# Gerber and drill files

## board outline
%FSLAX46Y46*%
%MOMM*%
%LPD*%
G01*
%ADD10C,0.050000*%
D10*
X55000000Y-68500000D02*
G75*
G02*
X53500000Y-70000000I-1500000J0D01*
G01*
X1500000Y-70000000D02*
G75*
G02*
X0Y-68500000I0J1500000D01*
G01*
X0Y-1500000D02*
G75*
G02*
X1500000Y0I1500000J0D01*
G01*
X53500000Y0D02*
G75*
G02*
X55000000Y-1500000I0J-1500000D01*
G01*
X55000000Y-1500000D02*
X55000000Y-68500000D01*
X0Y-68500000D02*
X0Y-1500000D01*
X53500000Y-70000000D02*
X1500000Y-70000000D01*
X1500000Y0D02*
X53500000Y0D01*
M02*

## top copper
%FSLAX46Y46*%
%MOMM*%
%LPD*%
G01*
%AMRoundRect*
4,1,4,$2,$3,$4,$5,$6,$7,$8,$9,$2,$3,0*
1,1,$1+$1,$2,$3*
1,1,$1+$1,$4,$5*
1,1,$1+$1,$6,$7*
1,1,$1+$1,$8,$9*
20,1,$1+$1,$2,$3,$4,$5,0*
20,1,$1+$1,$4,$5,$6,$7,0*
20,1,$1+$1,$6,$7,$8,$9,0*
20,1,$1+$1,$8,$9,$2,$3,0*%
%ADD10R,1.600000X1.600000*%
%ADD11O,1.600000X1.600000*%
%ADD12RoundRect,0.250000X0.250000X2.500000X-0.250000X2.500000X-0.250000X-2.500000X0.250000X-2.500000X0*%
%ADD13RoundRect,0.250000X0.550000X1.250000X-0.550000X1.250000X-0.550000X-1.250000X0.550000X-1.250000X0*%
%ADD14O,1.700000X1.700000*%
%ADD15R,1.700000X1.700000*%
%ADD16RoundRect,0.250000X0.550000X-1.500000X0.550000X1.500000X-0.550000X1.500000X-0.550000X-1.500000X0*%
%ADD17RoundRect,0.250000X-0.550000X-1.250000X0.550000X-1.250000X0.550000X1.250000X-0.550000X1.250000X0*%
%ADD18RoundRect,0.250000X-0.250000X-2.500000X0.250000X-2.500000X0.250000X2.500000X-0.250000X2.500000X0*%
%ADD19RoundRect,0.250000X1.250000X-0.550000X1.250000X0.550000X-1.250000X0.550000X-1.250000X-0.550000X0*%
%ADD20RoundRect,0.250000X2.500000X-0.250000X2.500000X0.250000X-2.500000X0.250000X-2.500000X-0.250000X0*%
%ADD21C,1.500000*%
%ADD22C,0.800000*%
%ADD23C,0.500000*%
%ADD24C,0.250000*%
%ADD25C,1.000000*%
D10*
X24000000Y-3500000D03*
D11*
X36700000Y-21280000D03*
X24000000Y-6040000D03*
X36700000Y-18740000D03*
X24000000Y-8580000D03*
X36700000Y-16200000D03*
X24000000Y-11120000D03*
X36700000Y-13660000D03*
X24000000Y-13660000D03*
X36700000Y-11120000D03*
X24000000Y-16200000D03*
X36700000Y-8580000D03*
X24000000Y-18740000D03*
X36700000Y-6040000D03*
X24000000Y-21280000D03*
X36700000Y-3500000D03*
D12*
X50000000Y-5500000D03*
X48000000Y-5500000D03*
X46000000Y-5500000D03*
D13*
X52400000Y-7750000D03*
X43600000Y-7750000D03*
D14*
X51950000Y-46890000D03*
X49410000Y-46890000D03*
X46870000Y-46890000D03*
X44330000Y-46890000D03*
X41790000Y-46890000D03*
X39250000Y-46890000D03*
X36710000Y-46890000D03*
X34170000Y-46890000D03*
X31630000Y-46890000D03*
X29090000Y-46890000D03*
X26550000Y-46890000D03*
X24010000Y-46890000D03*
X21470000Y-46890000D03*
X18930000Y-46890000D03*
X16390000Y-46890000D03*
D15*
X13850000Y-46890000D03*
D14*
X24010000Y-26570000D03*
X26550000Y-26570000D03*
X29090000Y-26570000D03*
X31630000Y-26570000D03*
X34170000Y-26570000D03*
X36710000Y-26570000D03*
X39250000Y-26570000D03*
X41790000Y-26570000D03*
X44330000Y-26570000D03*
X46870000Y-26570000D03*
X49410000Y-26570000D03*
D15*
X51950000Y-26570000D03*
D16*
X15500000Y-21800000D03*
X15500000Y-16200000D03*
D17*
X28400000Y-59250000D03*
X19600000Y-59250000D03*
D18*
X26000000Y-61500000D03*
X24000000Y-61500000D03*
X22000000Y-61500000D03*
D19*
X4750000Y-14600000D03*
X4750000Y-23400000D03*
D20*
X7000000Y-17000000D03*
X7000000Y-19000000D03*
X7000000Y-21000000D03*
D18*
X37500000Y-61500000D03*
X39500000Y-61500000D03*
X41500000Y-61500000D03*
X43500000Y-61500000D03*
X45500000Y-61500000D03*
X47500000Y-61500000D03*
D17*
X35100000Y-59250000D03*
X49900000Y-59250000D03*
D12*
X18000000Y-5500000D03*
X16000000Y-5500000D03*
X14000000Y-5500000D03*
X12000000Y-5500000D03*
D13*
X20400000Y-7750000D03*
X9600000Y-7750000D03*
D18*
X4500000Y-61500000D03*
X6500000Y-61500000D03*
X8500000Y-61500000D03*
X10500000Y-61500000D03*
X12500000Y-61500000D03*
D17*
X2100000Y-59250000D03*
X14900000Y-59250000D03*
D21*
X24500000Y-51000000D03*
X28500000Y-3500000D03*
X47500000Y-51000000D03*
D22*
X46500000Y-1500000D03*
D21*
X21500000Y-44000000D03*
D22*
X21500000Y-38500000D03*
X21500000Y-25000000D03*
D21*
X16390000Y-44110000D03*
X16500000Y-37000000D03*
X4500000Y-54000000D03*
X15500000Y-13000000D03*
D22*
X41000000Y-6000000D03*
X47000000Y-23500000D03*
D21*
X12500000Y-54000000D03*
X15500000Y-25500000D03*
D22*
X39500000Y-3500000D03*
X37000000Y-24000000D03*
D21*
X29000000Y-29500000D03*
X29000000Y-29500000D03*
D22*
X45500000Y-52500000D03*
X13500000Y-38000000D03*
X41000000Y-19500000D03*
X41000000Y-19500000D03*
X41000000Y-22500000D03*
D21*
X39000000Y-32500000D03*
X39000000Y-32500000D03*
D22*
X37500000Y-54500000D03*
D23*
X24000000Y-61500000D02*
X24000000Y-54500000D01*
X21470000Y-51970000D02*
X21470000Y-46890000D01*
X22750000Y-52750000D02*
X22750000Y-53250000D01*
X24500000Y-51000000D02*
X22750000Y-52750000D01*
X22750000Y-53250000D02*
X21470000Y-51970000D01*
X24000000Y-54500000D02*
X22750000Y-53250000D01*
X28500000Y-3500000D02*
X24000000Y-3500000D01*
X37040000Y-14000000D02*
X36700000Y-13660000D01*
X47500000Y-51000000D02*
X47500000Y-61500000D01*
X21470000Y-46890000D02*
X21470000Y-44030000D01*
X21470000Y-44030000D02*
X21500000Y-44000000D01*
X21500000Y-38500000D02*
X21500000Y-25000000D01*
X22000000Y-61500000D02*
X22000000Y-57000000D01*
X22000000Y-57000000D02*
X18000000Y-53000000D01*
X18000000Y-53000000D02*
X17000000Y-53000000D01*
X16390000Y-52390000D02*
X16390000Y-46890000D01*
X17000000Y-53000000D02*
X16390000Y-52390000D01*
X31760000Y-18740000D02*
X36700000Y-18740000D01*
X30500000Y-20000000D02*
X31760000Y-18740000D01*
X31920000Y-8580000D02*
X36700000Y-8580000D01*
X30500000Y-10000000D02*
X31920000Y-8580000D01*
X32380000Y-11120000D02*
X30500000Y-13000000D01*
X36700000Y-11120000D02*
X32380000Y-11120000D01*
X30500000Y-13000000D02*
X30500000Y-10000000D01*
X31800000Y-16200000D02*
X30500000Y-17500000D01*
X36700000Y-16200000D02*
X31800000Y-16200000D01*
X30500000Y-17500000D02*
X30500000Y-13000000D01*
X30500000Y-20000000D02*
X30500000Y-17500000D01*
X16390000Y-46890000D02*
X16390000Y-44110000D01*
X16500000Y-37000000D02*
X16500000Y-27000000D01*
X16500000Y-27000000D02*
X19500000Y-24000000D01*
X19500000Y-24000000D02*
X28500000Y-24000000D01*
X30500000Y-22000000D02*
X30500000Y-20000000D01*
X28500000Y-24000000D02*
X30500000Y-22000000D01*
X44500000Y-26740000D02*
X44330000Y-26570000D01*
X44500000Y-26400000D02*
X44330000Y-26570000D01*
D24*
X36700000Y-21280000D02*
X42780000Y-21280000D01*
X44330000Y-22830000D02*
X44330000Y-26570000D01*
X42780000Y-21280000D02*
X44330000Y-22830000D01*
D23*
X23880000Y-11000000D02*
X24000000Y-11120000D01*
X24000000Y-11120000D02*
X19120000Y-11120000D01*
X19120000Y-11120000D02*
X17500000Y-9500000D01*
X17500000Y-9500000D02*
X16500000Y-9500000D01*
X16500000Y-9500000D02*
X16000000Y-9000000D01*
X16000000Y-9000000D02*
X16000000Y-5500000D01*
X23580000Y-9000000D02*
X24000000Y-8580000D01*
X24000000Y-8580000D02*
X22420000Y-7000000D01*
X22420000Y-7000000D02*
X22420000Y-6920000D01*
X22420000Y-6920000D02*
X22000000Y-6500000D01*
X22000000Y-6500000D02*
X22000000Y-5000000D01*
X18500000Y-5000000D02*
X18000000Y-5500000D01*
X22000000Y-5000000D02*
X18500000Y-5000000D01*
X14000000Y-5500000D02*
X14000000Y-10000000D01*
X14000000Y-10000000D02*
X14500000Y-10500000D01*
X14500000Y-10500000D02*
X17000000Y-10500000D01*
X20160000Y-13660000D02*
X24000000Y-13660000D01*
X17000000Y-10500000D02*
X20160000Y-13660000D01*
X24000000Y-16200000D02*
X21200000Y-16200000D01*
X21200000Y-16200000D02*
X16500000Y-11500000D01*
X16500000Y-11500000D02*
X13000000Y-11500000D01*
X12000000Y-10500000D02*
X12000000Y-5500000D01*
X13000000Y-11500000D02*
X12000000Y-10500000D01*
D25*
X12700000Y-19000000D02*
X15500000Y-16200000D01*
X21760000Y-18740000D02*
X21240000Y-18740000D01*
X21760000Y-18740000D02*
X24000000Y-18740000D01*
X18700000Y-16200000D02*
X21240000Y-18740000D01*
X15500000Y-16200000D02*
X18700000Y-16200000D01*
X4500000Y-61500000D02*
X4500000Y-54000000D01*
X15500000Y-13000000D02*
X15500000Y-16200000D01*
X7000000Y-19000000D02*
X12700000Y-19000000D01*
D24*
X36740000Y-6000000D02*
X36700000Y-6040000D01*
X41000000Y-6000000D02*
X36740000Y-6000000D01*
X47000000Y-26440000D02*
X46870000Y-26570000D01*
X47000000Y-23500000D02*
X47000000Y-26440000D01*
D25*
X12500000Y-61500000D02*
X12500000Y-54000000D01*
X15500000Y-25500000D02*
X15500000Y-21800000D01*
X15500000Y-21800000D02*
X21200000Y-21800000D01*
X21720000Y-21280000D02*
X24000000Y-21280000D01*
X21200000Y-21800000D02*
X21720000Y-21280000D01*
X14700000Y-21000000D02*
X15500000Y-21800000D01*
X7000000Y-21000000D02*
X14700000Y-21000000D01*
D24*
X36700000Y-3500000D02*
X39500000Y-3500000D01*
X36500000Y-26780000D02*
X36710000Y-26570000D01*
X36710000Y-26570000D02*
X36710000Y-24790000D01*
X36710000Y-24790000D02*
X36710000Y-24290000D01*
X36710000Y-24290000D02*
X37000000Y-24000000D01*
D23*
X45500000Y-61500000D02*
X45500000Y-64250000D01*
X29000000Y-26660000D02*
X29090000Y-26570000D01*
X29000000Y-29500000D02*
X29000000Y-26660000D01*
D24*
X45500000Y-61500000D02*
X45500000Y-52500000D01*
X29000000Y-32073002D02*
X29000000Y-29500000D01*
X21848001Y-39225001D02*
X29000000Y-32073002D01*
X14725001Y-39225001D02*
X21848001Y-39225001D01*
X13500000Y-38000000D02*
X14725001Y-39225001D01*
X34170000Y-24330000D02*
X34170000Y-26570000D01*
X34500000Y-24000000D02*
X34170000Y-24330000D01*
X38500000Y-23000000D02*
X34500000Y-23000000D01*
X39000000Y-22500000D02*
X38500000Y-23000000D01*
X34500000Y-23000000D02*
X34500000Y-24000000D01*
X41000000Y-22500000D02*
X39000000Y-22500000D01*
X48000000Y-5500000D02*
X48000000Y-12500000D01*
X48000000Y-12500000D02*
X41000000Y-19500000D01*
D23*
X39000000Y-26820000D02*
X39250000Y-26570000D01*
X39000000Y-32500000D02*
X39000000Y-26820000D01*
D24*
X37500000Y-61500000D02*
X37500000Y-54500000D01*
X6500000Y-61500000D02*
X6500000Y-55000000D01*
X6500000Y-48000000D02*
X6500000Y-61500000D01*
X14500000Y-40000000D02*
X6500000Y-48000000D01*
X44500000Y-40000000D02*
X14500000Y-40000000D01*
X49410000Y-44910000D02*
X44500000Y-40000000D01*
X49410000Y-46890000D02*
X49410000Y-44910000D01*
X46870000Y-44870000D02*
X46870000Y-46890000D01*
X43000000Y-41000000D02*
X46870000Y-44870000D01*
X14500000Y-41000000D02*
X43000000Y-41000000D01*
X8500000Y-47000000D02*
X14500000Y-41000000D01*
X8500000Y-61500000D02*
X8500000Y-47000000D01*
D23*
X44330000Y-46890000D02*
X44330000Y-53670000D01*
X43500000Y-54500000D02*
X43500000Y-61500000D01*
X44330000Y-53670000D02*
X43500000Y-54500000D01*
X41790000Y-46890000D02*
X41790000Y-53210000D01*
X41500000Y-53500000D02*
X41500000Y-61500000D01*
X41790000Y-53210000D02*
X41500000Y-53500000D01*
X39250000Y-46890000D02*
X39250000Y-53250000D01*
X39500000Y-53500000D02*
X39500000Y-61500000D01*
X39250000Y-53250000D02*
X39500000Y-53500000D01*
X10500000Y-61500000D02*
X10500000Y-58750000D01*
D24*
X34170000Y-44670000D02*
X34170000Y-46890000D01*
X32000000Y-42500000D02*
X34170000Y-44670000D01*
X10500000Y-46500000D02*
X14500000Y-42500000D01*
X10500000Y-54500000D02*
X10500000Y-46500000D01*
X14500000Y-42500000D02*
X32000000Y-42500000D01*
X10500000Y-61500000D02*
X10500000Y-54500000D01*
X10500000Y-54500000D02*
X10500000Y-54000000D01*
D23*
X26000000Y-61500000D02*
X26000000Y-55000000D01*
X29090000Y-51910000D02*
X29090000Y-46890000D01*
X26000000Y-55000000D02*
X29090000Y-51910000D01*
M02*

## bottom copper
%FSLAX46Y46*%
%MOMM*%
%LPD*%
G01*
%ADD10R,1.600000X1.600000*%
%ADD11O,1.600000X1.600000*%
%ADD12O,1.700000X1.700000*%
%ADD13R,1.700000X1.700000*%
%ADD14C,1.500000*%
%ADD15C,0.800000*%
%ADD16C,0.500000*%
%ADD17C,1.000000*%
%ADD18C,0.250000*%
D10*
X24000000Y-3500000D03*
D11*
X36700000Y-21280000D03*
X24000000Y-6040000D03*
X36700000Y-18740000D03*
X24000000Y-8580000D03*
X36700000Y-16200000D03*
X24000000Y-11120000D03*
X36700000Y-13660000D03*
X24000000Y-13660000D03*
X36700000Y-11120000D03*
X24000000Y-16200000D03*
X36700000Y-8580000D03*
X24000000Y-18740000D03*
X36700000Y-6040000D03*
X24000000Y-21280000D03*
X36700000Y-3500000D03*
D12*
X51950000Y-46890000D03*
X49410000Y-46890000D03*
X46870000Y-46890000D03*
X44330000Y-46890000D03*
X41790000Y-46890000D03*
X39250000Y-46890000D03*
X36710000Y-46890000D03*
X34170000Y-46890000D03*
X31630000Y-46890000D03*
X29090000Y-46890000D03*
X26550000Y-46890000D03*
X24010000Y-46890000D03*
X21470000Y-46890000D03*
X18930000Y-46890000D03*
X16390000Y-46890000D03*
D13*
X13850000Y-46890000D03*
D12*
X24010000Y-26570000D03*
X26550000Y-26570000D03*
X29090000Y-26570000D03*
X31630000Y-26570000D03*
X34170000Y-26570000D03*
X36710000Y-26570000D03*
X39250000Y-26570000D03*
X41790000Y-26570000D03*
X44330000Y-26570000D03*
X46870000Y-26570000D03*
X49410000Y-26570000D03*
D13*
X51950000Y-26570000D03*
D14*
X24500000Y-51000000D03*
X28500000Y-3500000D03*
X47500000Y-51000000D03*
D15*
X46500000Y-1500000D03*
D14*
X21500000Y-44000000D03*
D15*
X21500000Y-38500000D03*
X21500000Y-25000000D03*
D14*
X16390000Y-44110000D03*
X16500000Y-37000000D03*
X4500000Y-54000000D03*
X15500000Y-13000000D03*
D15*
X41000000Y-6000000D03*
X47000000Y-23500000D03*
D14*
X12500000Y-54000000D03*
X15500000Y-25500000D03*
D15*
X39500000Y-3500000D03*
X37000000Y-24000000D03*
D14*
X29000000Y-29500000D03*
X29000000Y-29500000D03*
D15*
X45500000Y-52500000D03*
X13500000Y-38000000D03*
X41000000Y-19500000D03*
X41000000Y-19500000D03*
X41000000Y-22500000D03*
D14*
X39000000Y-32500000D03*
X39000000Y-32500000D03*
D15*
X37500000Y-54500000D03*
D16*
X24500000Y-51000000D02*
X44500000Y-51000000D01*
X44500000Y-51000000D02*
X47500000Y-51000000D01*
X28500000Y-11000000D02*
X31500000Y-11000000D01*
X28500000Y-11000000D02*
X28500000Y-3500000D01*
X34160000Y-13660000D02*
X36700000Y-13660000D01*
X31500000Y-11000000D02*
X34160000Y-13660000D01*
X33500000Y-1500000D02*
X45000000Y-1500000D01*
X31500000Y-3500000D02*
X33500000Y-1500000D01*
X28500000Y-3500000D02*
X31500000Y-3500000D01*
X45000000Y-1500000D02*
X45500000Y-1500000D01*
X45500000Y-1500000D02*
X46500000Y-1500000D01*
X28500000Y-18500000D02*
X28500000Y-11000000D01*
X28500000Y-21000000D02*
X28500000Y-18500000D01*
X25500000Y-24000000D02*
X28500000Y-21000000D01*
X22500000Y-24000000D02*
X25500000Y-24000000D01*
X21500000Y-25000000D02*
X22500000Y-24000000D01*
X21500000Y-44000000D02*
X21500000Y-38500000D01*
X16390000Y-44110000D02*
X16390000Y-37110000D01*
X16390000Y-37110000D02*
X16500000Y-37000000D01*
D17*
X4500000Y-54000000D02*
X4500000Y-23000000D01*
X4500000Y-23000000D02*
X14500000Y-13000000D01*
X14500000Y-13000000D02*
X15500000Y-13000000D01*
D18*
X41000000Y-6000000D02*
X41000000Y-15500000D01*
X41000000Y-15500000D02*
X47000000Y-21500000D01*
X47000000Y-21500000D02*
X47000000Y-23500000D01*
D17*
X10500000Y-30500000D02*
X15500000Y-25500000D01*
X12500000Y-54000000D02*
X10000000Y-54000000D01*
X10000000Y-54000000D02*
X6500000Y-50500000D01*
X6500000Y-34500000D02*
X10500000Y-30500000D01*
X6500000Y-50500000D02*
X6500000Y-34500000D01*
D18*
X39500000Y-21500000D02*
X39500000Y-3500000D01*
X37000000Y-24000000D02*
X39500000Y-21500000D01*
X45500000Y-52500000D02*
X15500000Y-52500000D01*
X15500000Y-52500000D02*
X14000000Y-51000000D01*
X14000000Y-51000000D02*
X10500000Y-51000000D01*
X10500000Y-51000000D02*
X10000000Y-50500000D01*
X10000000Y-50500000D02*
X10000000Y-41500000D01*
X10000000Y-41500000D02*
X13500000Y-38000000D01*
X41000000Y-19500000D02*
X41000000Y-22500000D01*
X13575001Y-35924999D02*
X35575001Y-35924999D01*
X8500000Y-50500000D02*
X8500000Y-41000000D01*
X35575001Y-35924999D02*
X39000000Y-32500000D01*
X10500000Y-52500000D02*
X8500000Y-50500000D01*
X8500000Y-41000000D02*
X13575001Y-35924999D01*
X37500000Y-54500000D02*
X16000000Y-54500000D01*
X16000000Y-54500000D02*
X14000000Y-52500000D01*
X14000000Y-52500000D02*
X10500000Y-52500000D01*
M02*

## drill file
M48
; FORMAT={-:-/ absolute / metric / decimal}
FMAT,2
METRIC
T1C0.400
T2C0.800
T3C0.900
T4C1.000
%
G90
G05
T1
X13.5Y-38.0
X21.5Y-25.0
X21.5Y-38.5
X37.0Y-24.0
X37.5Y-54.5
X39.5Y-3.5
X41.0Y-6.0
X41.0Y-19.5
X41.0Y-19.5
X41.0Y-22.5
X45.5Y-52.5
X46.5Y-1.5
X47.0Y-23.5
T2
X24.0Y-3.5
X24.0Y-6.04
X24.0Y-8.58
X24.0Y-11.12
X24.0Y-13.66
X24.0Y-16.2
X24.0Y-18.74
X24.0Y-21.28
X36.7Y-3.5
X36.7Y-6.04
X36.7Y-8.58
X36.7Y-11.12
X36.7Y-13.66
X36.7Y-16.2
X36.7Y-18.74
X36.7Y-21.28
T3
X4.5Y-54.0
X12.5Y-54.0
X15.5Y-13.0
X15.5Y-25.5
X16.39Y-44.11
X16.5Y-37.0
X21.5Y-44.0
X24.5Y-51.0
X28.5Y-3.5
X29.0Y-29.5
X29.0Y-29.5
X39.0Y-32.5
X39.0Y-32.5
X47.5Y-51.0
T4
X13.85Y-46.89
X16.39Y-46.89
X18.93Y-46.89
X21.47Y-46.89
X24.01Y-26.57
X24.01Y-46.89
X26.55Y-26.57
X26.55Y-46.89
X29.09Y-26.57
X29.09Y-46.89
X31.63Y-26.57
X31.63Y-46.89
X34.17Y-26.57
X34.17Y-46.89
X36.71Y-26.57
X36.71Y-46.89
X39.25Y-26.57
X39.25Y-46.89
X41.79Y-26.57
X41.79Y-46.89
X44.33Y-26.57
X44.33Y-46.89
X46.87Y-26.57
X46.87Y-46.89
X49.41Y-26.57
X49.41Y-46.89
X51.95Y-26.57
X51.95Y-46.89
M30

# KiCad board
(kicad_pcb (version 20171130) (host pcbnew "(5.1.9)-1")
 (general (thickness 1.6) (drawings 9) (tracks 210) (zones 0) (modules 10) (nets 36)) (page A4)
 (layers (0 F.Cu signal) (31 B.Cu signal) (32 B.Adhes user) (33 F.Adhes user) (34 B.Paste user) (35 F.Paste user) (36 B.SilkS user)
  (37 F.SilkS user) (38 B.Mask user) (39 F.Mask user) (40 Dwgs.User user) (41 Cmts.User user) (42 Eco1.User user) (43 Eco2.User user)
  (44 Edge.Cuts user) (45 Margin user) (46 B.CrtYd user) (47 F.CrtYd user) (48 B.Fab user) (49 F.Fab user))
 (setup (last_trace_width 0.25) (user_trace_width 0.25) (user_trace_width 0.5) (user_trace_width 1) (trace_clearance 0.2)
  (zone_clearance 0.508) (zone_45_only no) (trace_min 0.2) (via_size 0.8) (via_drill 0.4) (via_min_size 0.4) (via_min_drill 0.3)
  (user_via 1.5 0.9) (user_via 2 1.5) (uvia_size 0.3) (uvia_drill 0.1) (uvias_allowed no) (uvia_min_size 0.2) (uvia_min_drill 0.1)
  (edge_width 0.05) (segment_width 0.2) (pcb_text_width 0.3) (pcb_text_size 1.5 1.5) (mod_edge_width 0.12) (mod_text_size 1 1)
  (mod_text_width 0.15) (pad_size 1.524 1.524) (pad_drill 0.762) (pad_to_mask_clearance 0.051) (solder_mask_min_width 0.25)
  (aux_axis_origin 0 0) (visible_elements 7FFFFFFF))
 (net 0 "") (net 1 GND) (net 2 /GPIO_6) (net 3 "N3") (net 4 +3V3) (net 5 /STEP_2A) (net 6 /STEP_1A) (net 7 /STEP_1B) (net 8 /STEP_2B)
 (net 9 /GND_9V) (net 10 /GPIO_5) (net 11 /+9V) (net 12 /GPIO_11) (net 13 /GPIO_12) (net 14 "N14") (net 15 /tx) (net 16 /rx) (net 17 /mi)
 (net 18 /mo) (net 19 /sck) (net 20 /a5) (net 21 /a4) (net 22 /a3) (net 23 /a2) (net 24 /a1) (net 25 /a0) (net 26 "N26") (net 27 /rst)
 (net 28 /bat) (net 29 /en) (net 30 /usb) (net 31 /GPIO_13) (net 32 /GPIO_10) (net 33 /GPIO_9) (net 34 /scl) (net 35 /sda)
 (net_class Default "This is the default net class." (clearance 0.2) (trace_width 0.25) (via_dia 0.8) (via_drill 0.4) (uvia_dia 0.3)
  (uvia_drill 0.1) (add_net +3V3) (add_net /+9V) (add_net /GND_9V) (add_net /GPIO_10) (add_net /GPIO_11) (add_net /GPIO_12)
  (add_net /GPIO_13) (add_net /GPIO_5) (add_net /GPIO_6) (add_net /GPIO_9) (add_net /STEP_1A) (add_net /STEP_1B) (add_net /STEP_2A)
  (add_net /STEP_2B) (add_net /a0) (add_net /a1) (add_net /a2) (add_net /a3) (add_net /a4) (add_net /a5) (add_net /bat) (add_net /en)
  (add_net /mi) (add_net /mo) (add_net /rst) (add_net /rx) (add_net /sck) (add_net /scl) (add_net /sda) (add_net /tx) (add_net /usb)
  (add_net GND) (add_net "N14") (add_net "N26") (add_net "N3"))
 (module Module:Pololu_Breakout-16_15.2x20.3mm (layer F.Cu) (at 24 3.5)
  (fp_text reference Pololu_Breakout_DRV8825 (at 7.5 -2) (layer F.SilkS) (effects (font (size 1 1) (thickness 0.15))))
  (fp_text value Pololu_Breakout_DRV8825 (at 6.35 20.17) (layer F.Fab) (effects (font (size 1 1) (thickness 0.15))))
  (pad 1 thru_hole rect (at 0 0) (size 1.6 1.6) (drill 0.8) (layers *.Cu *.Mask) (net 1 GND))
  (pad 9 thru_hole oval (at 12.7 17.78) (size 1.6 1.6) (drill 0.8) (layers *.Cu *.Mask) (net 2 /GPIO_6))
  (pad 2 thru_hole oval (at 0 2.54) (size 1.6 1.6) (drill 0.8) (layers *.Cu *.Mask) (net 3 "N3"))
  (pad 10 thru_hole oval (at 12.7 15.24) (size 1.6 1.6) (drill 0.8) (layers *.Cu *.Mask) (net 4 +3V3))
  (pad 3 thru_hole oval (at 0 5.08) (size 1.6 1.6) (drill 0.8) (layers *.Cu *.Mask) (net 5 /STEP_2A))
  (pad 11 thru_hole oval (at 12.7 12.7) (size 1.6 1.6) (drill 0.8) (layers *.Cu *.Mask) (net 4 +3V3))
  (pad 4 thru_hole oval (at 0 7.62) (size 1.6 1.6) (drill 0.8) (layers *.Cu *.Mask) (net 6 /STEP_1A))
  (pad 12 thru_hole oval (at 12.7 10.16) (size 1.6 1.6) (drill 0.8) (layers *.Cu *.Mask) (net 1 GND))
  (pad 5 thru_hole oval (at 0 10.16) (size 1.6 1.6) (drill 0.8) (layers *.Cu *.Mask) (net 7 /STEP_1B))
  (pad 13 thru_hole oval (at 12.7 7.62) (size 1.6 1.6) (drill 0.8) (layers *.Cu *.Mask) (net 4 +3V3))
  (pad 6 thru_hole oval (at 0 12.7) (size 1.6 1.6) (drill 0.8) (layers *.Cu *.Mask) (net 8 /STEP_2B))
  (pad 14 thru_hole oval (at 12.7 5.08) (size 1.6 1.6) (drill 0.8) (layers *.Cu *.Mask) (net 4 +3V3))
  (pad 7 thru_hole oval (at 0 15.24) (size 1.6 1.6) (drill 0.8) (layers *.Cu *.Mask) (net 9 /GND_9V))
  (pad 15 thru_hole oval (at 12.7 2.54) (size 1.6 1.6) (drill 0.8) (layers *.Cu *.Mask) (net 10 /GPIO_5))
  (pad 8 thru_hole oval (at 0 17.78) (size 1.6 1.6) (drill 0.8) (layers *.Cu *.Mask) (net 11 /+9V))
  (pad 16 thru_hole oval (at 12.7 0) (size 1.6 1.6) (drill 0.8) (layers *.Cu *.Mask) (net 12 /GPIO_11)))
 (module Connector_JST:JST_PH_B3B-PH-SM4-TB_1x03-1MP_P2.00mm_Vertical (layer F.Cu) (at 48 6 180)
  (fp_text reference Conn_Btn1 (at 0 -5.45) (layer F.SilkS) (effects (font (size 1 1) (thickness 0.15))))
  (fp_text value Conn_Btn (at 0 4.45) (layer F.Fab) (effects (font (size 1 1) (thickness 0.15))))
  (pad 1 smd roundrect (at -2 0.5 180) (size 1 5.5) (layers F.Cu F.Paste F.Mask) (roundrect_rratio 0.25) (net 1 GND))
  (pad 2 smd roundrect (at 0 0.5 180) (size 1 5.5) (layers F.Cu F.Paste F.Mask) (roundrect_rratio 0.25) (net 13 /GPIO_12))
  (pad 3 smd roundrect (at 2 0.5 180) (size 1 5.5) (layers F.Cu F.Paste F.Mask) (roundrect_rratio 0.25))
  (pad MP smd roundrect (at -4.4 -1.75 180) (size 1.6 3) (layers F.Cu F.Paste F.Mask) (roundrect_rratio 0.15625))
  (pad MP smd roundrect (at 4.4 -1.75 180) (size 1.6 3) (layers F.Cu F.Paste F.Mask) (roundrect_rratio 0.15625)))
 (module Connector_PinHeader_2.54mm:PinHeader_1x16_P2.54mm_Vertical (layer F.Cu) (at 13.85 46.89 90)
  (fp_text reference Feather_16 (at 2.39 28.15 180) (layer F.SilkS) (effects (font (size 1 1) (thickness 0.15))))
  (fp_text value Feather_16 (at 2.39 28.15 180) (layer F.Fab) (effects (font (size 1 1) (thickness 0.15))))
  (pad 16 thru_hole oval (at 0 38.1 90) (size 1.7 1.7) (drill 1) (layers *.Cu *.Mask) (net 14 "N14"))
  (pad 15 thru_hole oval (at 0 35.56 90) (size 1.7 1.7) (drill 1) (layers *.Cu *.Mask) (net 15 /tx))
  (pad 14 thru_hole oval (at 0 33.02 90) (size 1.7 1.7) (drill 1) (layers *.Cu *.Mask) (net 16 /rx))
  (pad 13 thru_hole oval (at 0 30.48 90) (size 1.7 1.7) (drill 1) (layers *.Cu *.Mask) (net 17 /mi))
  (pad 12 thru_hole oval (at 0 27.94 90) (size 1.7 1.7) (drill 1) (layers *.Cu *.Mask) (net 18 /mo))
  (pad 11 thru_hole oval (at 0 25.4 90) (size 1.7 1.7) (drill 1) (layers *.Cu *.Mask) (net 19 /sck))
  (pad 10 thru_hole oval (at 0 22.86 90) (size 1.7 1.7) (drill 1) (layers *.Cu *.Mask) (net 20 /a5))
  (pad 9 thru_hole oval (at 0 20.32 90) (size 1.7 1.7) (drill 1) (layers *.Cu *.Mask) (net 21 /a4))
  (pad 8 thru_hole oval (at 0 17.78 90) (size 1.7 1.7) (drill 1) (layers *.Cu *.Mask) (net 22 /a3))
  (pad 7 thru_hole oval (at 0 15.24 90) (size 1.7 1.7) (drill 1) (layers *.Cu *.Mask) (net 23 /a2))
  (pad 6 thru_hole oval (at 0 12.7 90) (size 1.7 1.7) (drill 1) (layers *.Cu *.Mask) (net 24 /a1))
  (pad 5 thru_hole oval (at 0 10.16 90) (size 1.7 1.7) (drill 1) (layers *.Cu *.Mask) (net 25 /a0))
  (pad 4 thru_hole oval (at 0 7.62 90) (size 1.7 1.7) (drill 1) (layers *.Cu *.Mask) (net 1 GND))
  (pad 3 thru_hole oval (at 0 5.08 90) (size 1.7 1.7) (drill 1) (layers *.Cu *.Mask) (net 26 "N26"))
  (pad 2 thru_hole oval (at 0 2.54 90) (size 1.7 1.7) (drill 1) (layers *.Cu *.Mask) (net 4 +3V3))
  (pad 1 thru_hole rect (at 0 0 90) (size 1.7 1.7) (drill 1) (layers *.Cu *.Mask) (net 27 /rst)))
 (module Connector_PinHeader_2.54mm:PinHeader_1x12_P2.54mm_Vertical (layer F.Cu) (at 51.95 26.57 270)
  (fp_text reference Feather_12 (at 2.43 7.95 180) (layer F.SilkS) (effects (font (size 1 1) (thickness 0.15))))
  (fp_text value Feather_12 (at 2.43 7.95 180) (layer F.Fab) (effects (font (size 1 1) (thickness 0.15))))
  (pad 12 thru_hole oval (at 0 27.94 270) (size 1.7 1.7) (drill 1) (layers *.Cu *.Mask) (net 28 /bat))
  (pad 11 thru_hole oval (at 0 25.4 270) (size 1.7 1.7) (drill 1) (layers *.Cu *.Mask) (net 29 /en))
  (pad 10 thru_hole oval (at 0 22.86 270) (size 1.7 1.7) (drill 1) (layers *.Cu *.Mask) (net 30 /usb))
  (pad 9 thru_hole oval (at 0 20.32 270) (size 1.7 1.7) (drill 1) (layers *.Cu *.Mask) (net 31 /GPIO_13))
  (pad 8 thru_hole oval (at 0 17.78 270) (size 1.7 1.7) (drill 1) (layers *.Cu *.Mask) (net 13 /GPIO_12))
  (pad 7 thru_hole oval (at 0 15.24 270) (size 1.7 1.7) (drill 1) (layers *.Cu *.Mask) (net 12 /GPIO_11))
  (pad 6 thru_hole oval (at 0 12.7 270) (size 1.7 1.7) (drill 1) (layers *.Cu *.Mask) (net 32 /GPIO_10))
  (pad 5 thru_hole oval (at 0 10.16 270) (size 1.7 1.7) (drill 1) (layers *.Cu *.Mask) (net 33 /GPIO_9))
  (pad 4 thru_hole oval (at 0 7.62 270) (size 1.7 1.7) (drill 1) (layers *.Cu *.Mask) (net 2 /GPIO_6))
  (pad 3 thru_hole oval (at 0 5.08 270) (size 1.7 1.7) (drill 1) (layers *.Cu *.Mask) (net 10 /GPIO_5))
  (pad 2 thru_hole oval (at 0 2.54 270) (size 1.7 1.7) (drill 1) (layers *.Cu *.Mask) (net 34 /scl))
  (pad 1 thru_hole rect (at 0 0 270) (size 1.7 1.7) (drill 1) (layers *.Cu *.Mask) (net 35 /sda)))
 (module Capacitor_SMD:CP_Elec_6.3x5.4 (layer F.Cu) (at 15.5 19 90)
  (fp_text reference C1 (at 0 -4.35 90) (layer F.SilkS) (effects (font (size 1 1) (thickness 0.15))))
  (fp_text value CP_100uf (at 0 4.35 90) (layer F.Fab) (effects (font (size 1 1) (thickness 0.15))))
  (pad 1 smd roundrect (at -2.8 0 90) (size 3.5 1.6) (layers F.Cu F.Paste F.Mask) (roundrect_rratio 0.15625) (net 11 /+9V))
  (pad 2 smd roundrect (at 2.8 0 90) (size 3.5 1.6) (layers F.Cu F.Paste F.Mask) (roundrect_rratio 0.15625) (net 9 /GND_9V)))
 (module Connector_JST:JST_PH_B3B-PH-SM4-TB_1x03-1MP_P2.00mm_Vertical (layer F.Cu) (at 24 61)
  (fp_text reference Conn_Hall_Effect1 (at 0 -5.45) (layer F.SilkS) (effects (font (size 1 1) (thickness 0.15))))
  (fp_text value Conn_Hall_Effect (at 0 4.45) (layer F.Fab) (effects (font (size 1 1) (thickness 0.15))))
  (pad MP smd roundrect (at 4.4 -1.75) (size 1.6 3) (layers F.Cu F.Paste F.Mask) (roundrect_rratio 0.15625))
  (pad MP smd roundrect (at -4.4 -1.75) (size 1.6 3) (layers F.Cu F.Paste F.Mask) (roundrect_rratio 0.15625))
  (pad 3 smd roundrect (at 2 0.5) (size 1 5.5) (layers F.Cu F.Paste F.Mask) (roundrect_rratio 0.25) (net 23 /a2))
  (pad 2 smd roundrect (at 0 0.5) (size 1 5.5) (layers F.Cu F.Paste F.Mask) (roundrect_rratio 0.25) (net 1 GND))
  (pad 1 smd roundrect (at -2 0.5) (size 1 5.5) (layers F.Cu F.Paste F.Mask) (roundrect_rratio 0.25) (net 4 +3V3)))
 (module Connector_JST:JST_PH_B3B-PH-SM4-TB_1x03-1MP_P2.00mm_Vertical (layer F.Cu) (at 6.5 19 90)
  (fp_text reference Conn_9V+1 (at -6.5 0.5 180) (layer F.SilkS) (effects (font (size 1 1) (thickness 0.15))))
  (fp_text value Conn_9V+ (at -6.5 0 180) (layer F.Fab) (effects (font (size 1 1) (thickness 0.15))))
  (pad MP smd roundrect (at 4.4 -1.75 90) (size 1.6 3) (layers F.Cu F.Paste F.Mask) (roundrect_rratio 0.15625))
  (pad MP smd roundrect (at -4.4 -1.75 90) (size 1.6 3) (layers F.Cu F.Paste F.Mask) (roundrect_rratio 0.15625))
  (pad 3 smd roundrect (at 2 0.5 90) (size 1 5.5) (layers F.Cu F.Paste F.Mask) (roundrect_rratio 0.25))
  (pad 2 smd roundrect (at 0 0.5 90) (size 1 5.5) (layers F.Cu F.Paste F.Mask) (roundrect_rratio 0.25) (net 9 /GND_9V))
  (pad 1 smd roundrect (at -2 0.5 90) (size 1 5.5) (layers F.Cu F.Paste F.Mask) (roundrect_rratio 0.25) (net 11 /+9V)))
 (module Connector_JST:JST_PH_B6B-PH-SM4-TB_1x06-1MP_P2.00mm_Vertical (layer F.Cu) (at 42.5 61)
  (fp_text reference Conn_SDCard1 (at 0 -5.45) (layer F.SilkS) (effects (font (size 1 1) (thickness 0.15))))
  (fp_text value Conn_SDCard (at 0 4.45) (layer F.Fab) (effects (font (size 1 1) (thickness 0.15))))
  (pad 1 smd roundrect (at -5 0.5) (size 1 5.5) (layers F.Cu F.Paste F.Mask) (roundrect_rratio 0.25) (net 32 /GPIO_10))
  (pad 2 smd roundrect (at -3 0.5) (size 1 5.5) (layers F.Cu F.Paste F.Mask) (roundrect_rratio 0.25) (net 19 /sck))
  (pad 3 smd roundrect (at -1 0.5) (size 1 5.5) (layers F.Cu F.Paste F.Mask) (roundrect_rratio 0.25) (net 18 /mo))
  (pad 4 smd roundrect (at 1 0.5) (size 1 5.5) (layers F.Cu F.Paste F.Mask) (roundrect_rratio 0.25) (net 17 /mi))
  (pad 5 smd roundrect (at 3 0.5) (size 1 5.5) (layers F.Cu F.Paste F.Mask) (roundrect_rratio 0.25) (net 30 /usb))
  (pad 6 smd roundrect (at 5 0.5) (size 1 5.5) (layers F.Cu F.Paste F.Mask) (roundrect_rratio 0.25) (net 1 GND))
  (pad MP smd roundrect (at -7.4 -1.75) (size 1.6 3) (layers F.Cu F.Paste F.Mask) (roundrect_rratio 0.15625))
  (pad MP smd roundrect (at 7.4 -1.75) (size 1.6 3) (layers F.Cu F.Paste F.Mask) (roundrect_rratio 0.15625)))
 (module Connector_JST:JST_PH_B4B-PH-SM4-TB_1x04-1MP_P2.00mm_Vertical (layer F.Cu) (at 15 6 180)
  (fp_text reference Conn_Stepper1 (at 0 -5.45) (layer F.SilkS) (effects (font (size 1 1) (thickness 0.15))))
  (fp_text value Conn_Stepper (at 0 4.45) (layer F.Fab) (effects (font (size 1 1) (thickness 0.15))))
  (pad 1 smd roundrect (at -3 0.5 180) (size 1 5.5) (layers F.Cu F.Paste F.Mask) (roundrect_rratio 0.25) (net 5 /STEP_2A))
  (pad 2 smd roundrect (at -1 0.5 180) (size 1 5.5) (layers F.Cu F.Paste F.Mask) (roundrect_rratio 0.25) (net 6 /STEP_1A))
  (pad 3 smd roundrect (at 1 0.5 180) (size 1 5.5) (layers F.Cu F.Paste F.Mask) (roundrect_rratio 0.25) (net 7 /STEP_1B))
  (pad 4 smd roundrect (at 3 0.5 180) (size 1 5.5) (layers F.Cu F.Paste F.Mask) (roundrect_rratio 0.25) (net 8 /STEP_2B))
  (pad MP smd roundrect (at -5.4 -1.75 180) (size 1.6 3) (layers F.Cu F.Paste F.Mask) (roundrect_rratio 0.15625))
  (pad MP smd roundrect (at 5.4 -1.75 180) (size 1.6 3) (layers F.Cu F.Paste F.Mask) (roundrect_rratio 0.15625)))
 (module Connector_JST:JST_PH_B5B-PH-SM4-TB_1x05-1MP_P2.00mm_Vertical (layer F.Cu) (at 8.5 61)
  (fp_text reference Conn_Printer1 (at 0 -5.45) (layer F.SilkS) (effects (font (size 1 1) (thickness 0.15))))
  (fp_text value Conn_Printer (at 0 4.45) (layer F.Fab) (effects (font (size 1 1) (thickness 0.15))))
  (pad 1 smd roundrect (at -4 0.5) (size 1 5.5) (layers F.Cu F.Paste F.Mask) (roundrect_rratio 0.25) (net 9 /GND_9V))
  (pad 2 smd roundrect (at -2 0.5) (size 1 5.5) (layers F.Cu F.Paste F.Mask) (roundrect_rratio 0.25) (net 15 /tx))
  (pad 3 smd roundrect (at 0 0.5) (size 1 5.5) (layers F.Cu F.Paste F.Mask) (roundrect_rratio 0.25) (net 16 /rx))
  (pad 4 smd roundrect (at 2 0.5) (size 1 5.5) (layers F.Cu F.Paste F.Mask) (roundrect_rratio 0.25) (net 21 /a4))
  (pad 5 smd roundrect (at 4 0.5) (size 1 5.5) (layers F.Cu F.Paste F.Mask) (roundrect_rratio 0.25) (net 11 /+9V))
  (pad MP smd roundrect (at -6.4 -1.75) (size 1.6 3) (layers F.Cu F.Paste F.Mask) (roundrect_rratio 0.15625))
  (pad MP smd roundrect (at 6.4 -1.75) (size 1.6 3) (layers F.Cu F.Paste F.Mask) (roundrect_rratio 0.15625)))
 (gr_arc (start 53.5 68.5) (end 53.5 70) (angle -90) (layer Edge.Cuts) (width 0.05))
 (gr_arc (start 1.5 68.5) (end 0 68.5) (angle -90) (layer Edge.Cuts) (width 0.05))
 (gr_arc (start 1.5 1.5) (end 1.5 0) (angle -90) (layer Edge.Cuts) (width 0.05))
 (gr_arc (start 53.5 1.5) (end 55 1.5) (angle -90) (layer Edge.Cuts) (width 0.05))
 (gr_line (start 55 1.5) (end 55 68.5) (layer Edge.Cuts) (width 0.05))
 (gr_line (start 0 68.5) (end 0 1.5) (layer Edge.Cuts) (width 0.05))
 (gr_line (start 53.5 70) (end 1.5 70) (layer Edge.Cuts) (width 0.05))
 (gr_line (start 1.5 0) (end 53.5 0) (layer Edge.Cuts) (width 0.05))
 (segment (start 24 61.5) (end 24 54.5) (width 0.5) (layer F.Cu) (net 1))
 (segment (start 21.47 51.97) (end 21.47 46.89) (width 0.5) (layer F.Cu) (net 1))
 (via (at 24.5 51) (size 1.5) (drill 0.9) (layers F.Cu B.Cu) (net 1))
 (segment (start 22.75 52.75) (end 22.75 53.25) (width 0.5) (layer F.Cu) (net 1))
 (segment (start 24.5 51) (end 22.75 52.75) (width 0.5) (layer F.Cu) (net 1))
 (segment (start 22.75 53.25) (end 21.47 51.97) (width 0.5) (layer F.Cu) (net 1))
 (segment (start 24 54.5) (end 22.75 53.25) (width 0.5) (layer F.Cu) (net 1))
 (segment (start 24.5 51) (end 44.5 51) (width 0.5) (layer B.Cu) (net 1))
 (via (at 28.5 3.5) (size 1.5) (drill 0.9) (layers F.Cu B.Cu) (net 1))
 (segment (start 28.5 3.5) (end 24 3.5) (width 0.5) (layer F.Cu) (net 1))
 (segment (start 37.04 14) (end 36.7 13.66) (width 0.5) (layer F.Cu) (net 1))
 (segment (start 44.5 51) (end 47.5 51) (width 0.5) (layer B.Cu) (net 1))
 (via (at 47.5 51) (size 1.5) (drill 0.9) (layers F.Cu B.Cu) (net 1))
 (segment (start 47.5 51) (end 47.5 61.5) (width 0.5) (layer F.Cu) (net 1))
 (segment (start 28.5 11) (end 31.5 11) (width 0.5) (layer B.Cu) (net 1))
 (segment (start 28.5 11) (end 28.5 3.5) (width 0.5) (layer B.Cu) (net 1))
 (segment (start 34.16 13.66) (end 36.7 13.66) (width 0.5) (layer B.Cu) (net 1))
 (segment (start 31.5 11) (end 34.16 13.66) (width 0.5) (layer B.Cu) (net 1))
 (segment (start 33.5 1.5) (end 45 1.5) (width 0.5) (layer B.Cu) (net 1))
 (segment (start 31.5 3.5) (end 33.5 1.5) (width 0.5) (layer B.Cu) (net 1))
 (segment (start 28.5 3.5) (end 31.5 3.5) (width 0.5) (layer B.Cu) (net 1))
 (segment (start 45 1.5) (end 45.5 1.5) (width 0.5) (layer B.Cu) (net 1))
 (segment (start 45.5 1.5) (end 46.5 1.5) (width 0.5) (layer B.Cu) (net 1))
 (via (at 46.5 1.5) (size 0.8) (drill 0.4) (layers F.Cu B.Cu) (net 1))
 (segment (start 21.47 46.89) (end 21.47 44.03) (width 0.5) (layer F.Cu) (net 1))
 (via (at 21.5 44) (size 1.5) (drill 0.9) (layers F.Cu B.Cu) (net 1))
 (segment (start 21.47 44.03) (end 21.5 44) (width 0.5) (layer F.Cu) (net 1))
 (segment (start 28.5 18.5) (end 28.5 11) (width 0.5) (layer B.Cu) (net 1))
 (segment (start 28.5 21) (end 28.5 18.5) (width 0.5) (layer B.Cu) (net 1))
 (segment (start 25.5 24) (end 28.5 21) (width 0.5) (layer B.Cu) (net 1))
 (segment (start 22.5 24) (end 25.5 24) (width 0.5) (layer B.Cu) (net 1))
 (segment (start 21.5 25) (end 22.5 24) (width 0.5) (layer B.Cu) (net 1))
 (segment (start 21.5 44) (end 21.5 38.5) (width 0.5) (layer B.Cu) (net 1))
 (via (at 21.5 38.5) (size 0.8) (drill 0.4) (layers F.Cu B.Cu) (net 1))
 (segment (start 21.5 38.5) (end 21.5 25) (width 0.5) (layer F.Cu) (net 1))
 (via (at 21.5 25) (size 0.8) (drill 0.4) (layers F.Cu B.Cu) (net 1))
 (segment (start 22 61.5) (end 22 57) (width 0.5) (layer F.Cu) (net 4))
 (segment (start 22 57) (end 18 53) (width 0.5) (layer F.Cu) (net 4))
 (segment (start 18 53) (end 17 53) (width 0.5) (layer F.Cu) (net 4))
 (segment (start 16.39 52.39) (end 16.39 46.89) (width 0.5) (layer F.Cu) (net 4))
 (segment (start 17 53) (end 16.39 52.39) (width 0.5) (layer F.Cu) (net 4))
 (segment (start 31.76 18.74) (end 36.7 18.74) (width 0.5) (layer F.Cu) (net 4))
 (segment (start 30.5 20) (end 31.76 18.74) (width 0.5) (layer F.Cu) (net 4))
 (segment (start 31.92 8.58) (end 36.7 8.58) (width 0.5) (layer F.Cu) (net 4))
 (segment (start 30.5 10) (end 31.92 8.58) (width 0.5) (layer F.Cu) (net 4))
 (segment (start 32.38 11.12) (end 30.5 13) (width 0.5) (layer F.Cu) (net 4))
 (segment (start 36.7 11.12) (end 32.38 11.12) (width 0.5) (layer F.Cu) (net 4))
 (segment (start 30.5 13) (end 30.5 10) (width 0.5) (layer F.Cu) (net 4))
 (segment (start 31.8 16.2) (end 30.5 17.5) (width 0.5) (layer F.Cu) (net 4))
 (segment (start 36.7 16.2) (end 31.8 16.2) (width 0.5) (layer F.Cu) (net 4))
 (segment (start 30.5 17.5) (end 30.5 13) (width 0.5) (layer F.Cu) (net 4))
 (segment (start 30.5 20) (end 30.5 17.5) (width 0.5) (layer F.Cu) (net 4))
 (segment (start 16.39 46.89) (end 16.39 44.11) (width 0.5) (layer F.Cu) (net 4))
 (via (at 16.39 44.11) (size 1.5) (drill 0.9) (layers F.Cu B.Cu) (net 4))
 (segment (start 16.39 44.11) (end 16.39 37.11) (width 0.5) (layer B.Cu) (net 4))
 (via (at 16.5 37) (size 1.5) (drill 0.9) (layers F.Cu B.Cu) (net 4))
 (segment (start 16.39 37.11) (end 16.5 37) (width 0.5) (layer B.Cu) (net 4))
 (segment (start 16.5 37) (end 16.5 27) (width 0.5) (layer F.Cu) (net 4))
 (segment (start 16.5 27) (end 19.5 24) (width 0.5) (layer F.Cu) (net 4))
 (segment (start 19.5 24) (end 28.5 24) (width 0.5) (layer F.Cu) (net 4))
 (segment (start 30.5 22) (end 30.5 20) (width 0.5) (layer F.Cu) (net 4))
 (segment (start 28.5 24) (end 30.5 22) (width 0.5) (layer F.Cu) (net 4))
 (segment (start 44.5 26.74) (end 44.33 26.57) (width 0.5) (layer F.Cu) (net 2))
 (segment (start 44.5 26.4) (end 44.33 26.57) (width 0.5) (layer F.Cu) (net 2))
 (segment (start 36.7 21.28) (end 42.78 21.28) (width 0.25) (layer F.Cu) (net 2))
 (segment (start 44.33 22.83) (end 44.33 26.57) (width 0.25) (layer F.Cu) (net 2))
 (segment (start 42.78 21.28) (end 44.33 22.83) (width 0.25) (layer F.Cu) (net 2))
 (segment (start 23.88 11) (end 24 11.12) (width 0.5) (layer F.Cu) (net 6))
 (segment (start 24 11.12) (end 19.12 11.12) (width 0.5) (layer F.Cu) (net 6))
 (segment (start 19.12 11.12) (end 17.5 9.5) (width 0.5) (layer F.Cu) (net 6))
 (segment (start 17.5 9.5) (end 16.5 9.5) (width 0.5) (layer F.Cu) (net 6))
 (segment (start 16.5 9.5) (end 16 9) (width 0.5) (layer F.Cu) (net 6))
 (segment (start 16 9) (end 16 5.5) (width 0.5) (layer F.Cu) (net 6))
 (segment (start 23.58 9) (end 24 8.58) (width 0.5) (layer F.Cu) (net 5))
 (segment (start 24 8.58) (end 22.42 7) (width 0.5) (layer F.Cu) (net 5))
 (segment (start 22.42 7) (end 22.42 6.92) (width 0.5) (layer F.Cu) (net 5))
 (segment (start 22.42 6.92) (end 22 6.5) (width 0.5) (layer F.Cu) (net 5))
 (segment (start 22 6.5) (end 22 5) (width 0.5) (layer F.Cu) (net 5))
 (segment (start 18.5 5) (end 18 5.5) (width 0.5) (layer F.Cu) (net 5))
 (segment (start 22 5) (end 18.5 5) (width 0.5) (layer F.Cu) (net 5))
 (segment (start 14 5.5) (end 14 10) (width 0.5) (layer F.Cu) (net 7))
 (segment (start 14 10) (end 14.5 10.5) (width 0.5) (layer F.Cu) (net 7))
 (segment (start 14.5 10.5) (end 17 10.5) (width 0.5) (layer F.Cu) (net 7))
 (segment (start 20.16 13.66) (end 24 13.66) (width 0.5) (layer F.Cu) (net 7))
 (segment (start 17 10.5) (end 20.16 13.66) (width 0.5) (layer F.Cu) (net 7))
 (segment (start 24 16.2) (end 21.2 16.2) (width 0.5) (layer F.Cu) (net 8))
 (segment (start 21.2 16.2) (end 16.5 11.5) (width 0.5) (layer F.Cu) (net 8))
 (segment (start 16.5 11.5) (end 13 11.5) (width 0.5) (layer F.Cu) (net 8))
 (segment (start 12 10.5) (end 12 5.5) (width 0.5) (layer F.Cu) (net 8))
 (segment (start 13 11.5) (end 12 10.5) (width 0.5) (layer F.Cu) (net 8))
 (segment (start 12.7 19) (end 15.5 16.2) (width 1) (layer F.Cu) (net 9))
 (segment (start 21.76 18.74) (end 21.24 18.74) (width 1) (layer F.Cu) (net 9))
 (segment (start 21.76 18.74) (end 24 18.74) (width 1) (layer F.Cu) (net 9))
 (segment (start 18.7 16.2) (end 21.24 18.74) (width 1) (layer F.Cu) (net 9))
 (segment (start 15.5 16.2) (end 18.7 16.2) (width 1) (layer F.Cu) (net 9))
 (segment (start 4.5 61.5) (end 4.5 54) (width 1) (layer F.Cu) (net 9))
 (via (at 4.5 54) (size 1.5) (drill 0.9) (layers F.Cu B.Cu) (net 9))
 (segment (start 4.5 54) (end 4.5 23) (width 1) (layer B.Cu) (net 9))
 (segment (start 4.5 23) (end 14.5 13) (width 1) (layer B.Cu) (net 9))
 (segment (start 14.5 13) (end 15.5 13) (width 1) (layer B.Cu) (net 9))
 (via (at 15.5 13) (size 1.5) (drill 0.9) (layers F.Cu B.Cu) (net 9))
 (segment (start 15.5 13) (end 15.5 16.2) (width 1) (layer F.Cu) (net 9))
 (segment (start 7 19) (end 12.7 19) (width 1) (layer F.Cu) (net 9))
 (via (at 41 6) (size 0.8) (drill 0.4) (layers F.Cu B.Cu) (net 10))
 (segment (start 36.74 6) (end 36.7 6.04) (width 0.25) (layer F.Cu) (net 10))
 (segment (start 41 6) (end 36.74 6) (width 0.25) (layer F.Cu) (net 10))
 (segment (start 41 6) (end 41 15.5) (width 0.25) (layer B.Cu) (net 10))
 (segment (start 41 15.5) (end 47 21.5) (width 0.25) (layer B.Cu) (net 10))
 (via (at 47 23.5) (size 0.8) (drill 0.4) (layers F.Cu B.Cu) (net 10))
 (segment (start 47 21.5) (end 47 23.5) (width 0.25) (layer B.Cu) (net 10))
 (segment (start 47 26.44) (end 46.87 26.57) (width 0.25) (layer F.Cu) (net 10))
 (segment (start 47 23.5) (end 47 26.44) (width 0.25) (layer F.Cu) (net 10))
 (segment (start 12.5 61.5) (end 12.5 54) (width 1) (layer F.Cu) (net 11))
 (via (at 12.5 54) (size 1.5) (drill 0.9) (layers F.Cu B.Cu) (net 11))
 (via (at 15.5 25.5) (size 1.5) (drill 0.9) (layers F.Cu B.Cu) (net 11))
 (segment (start 10.5 30.5) (end 15.5 25.5) (width 1) (layer B.Cu) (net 11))
 (segment (start 15.5 25.5) (end 15.5 21.8) (width 1) (layer F.Cu) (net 11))
 (segment (start 15.5 21.8) (end 21.2 21.8) (width 1) (layer F.Cu) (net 11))
 (segment (start 21.72 21.28) (end 24 21.28) (width 1) (layer F.Cu) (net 11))
 (segment (start 21.2 21.8) (end 21.72 21.28) (width 1) (layer F.Cu) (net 11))
 (segment (start 12.5 54) (end 10 54) (width 1) (layer B.Cu) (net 11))
 (segment (start 10 54) (end 6.5 50.5) (width 1) (layer B.Cu) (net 11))
 (segment (start 6.5 34.5) (end 10.5 30.5) (width 1) (layer B.Cu) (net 11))
 (segment (start 6.5 50.5) (end 6.5 34.5) (width 1) (layer B.Cu) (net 11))
 (segment (start 14.7 21) (end 15.5 21.8) (width 1) (layer F.Cu) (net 11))
 (segment (start 7 21) (end 14.7 21) (width 1) (layer F.Cu) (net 11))
 (segment (start 36.7 3.5) (end 39.5 3.5) (width 0.25) (layer F.Cu) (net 12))
 (via (at 39.5 3.5) (size 0.8) (drill 0.4) (layers F.Cu B.Cu) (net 12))
 (segment (start 36.5 26.78) (end 36.71 26.57) (width 0.25) (layer F.Cu) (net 12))
 (segment (start 36.71 26.57) (end 36.71 24.79) (width 0.25) (layer F.Cu) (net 12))
 (segment (start 36.71 24.79) (end 36.71 24.29) (width 0.25) (layer F.Cu) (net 12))
 (via (at 37 24) (size 0.8) (drill 0.4) (layers F.Cu B.Cu) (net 12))
 (segment (start 36.71 24.29) (end 37 24) (width 0.25) (layer F.Cu) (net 12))
 (segment (start 39.5 21.5) (end 39.5 3.5) (width 0.25) (layer B.Cu) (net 12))
 (segment (start 37 24) (end 39.5 21.5) (width 0.25) (layer B.Cu) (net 12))
 (segment (start 45.5 61.5) (end 45.5 64.25) (width 0.5) (layer F.Cu) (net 30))
 (via (at 29 29.5) (size 1.5) (drill 0.9) (layers F.Cu B.Cu) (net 30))
 (via (at 29 29.5) (size 1.5) (drill 0.9) (layers F.Cu B.Cu) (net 30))
 (segment (start 29 26.66) (end 29.09 26.57) (width 0.5) (layer F.Cu) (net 30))
 (segment (start 29 29.5) (end 29 26.66) (width 0.5) (layer F.Cu) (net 30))
 (segment (start 45.5 61.5) (end 45.5 52.5) (width 0.25) (layer F.Cu) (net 30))
 (via (at 45.5 52.5) (size 0.8) (drill 0.4) (layers F.Cu B.Cu) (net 30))
 (segment (start 45.5 52.5) (end 15.5 52.5) (width 0.25) (layer B.Cu) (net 30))
 (segment (start 15.5 52.5) (end 14 51) (width 0.25) (layer B.Cu) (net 30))
 (segment (start 14 51) (end 10.5 51) (width 0.25) (layer B.Cu) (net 30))
 (segment (start 10.5 51) (end 10 50.5) (width 0.25) (layer B.Cu) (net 30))
 (segment (start 10 50.5) (end 10 41.5) (width 0.25) (layer B.Cu) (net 30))
 (via (at 13.5 38) (size 0.8) (drill 0.4) (layers F.Cu B.Cu) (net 30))
 (segment (start 10 41.5) (end 13.5 38) (width 0.25) (layer B.Cu) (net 30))
 (segment (start 29 32.073002) (end 29 29.5) (width 0.25) (layer F.Cu) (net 30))
 (segment (start 21.848001 39.225001) (end 29 32.073002) (width 0.25) (layer F.Cu) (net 30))
 (segment (start 14.725001 39.225001) (end 21.848001 39.225001) (width 0.25) (layer F.Cu) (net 30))
 (segment (start 13.5 38) (end 14.725001 39.225001) (width 0.25) (layer F.Cu) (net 30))
 (via (at 41 19.5) (size 0.8) (drill 0.4) (layers F.Cu B.Cu) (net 13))
 (via (at 41 19.5) (size 0.8) (drill 0.4) (layers F.Cu B.Cu) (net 13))
 (segment (start 41 19.5) (end 41 22.5) (width 0.25) (layer B.Cu) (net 13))
 (via (at 41 22.5) (size 0.8) (drill 0.4) (layers F.Cu B.Cu) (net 13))
 (segment (start 34.17 24.33) (end 34.17 26.57) (width 0.25) (layer F.Cu) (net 13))
 (segment (start 34.5 24) (end 34.17 24.33) (width 0.25) (layer F.Cu) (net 13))
 (segment (start 38.5 23) (end 34.5 23) (width 0.25) (layer F.Cu) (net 13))
 (segment (start 39 22.5) (end 38.5 23) (width 0.25) (layer F.Cu) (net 13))
 (segment (start 34.5 23) (end 34.5 24) (width 0.25) (layer F.Cu) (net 13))
 (segment (start 41 22.5) (end 39 22.5) (width 0.25) (layer F.Cu) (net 13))
 (segment (start 48 5.5) (end 48 12.5) (width 0.25) (layer F.Cu) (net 13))
 (segment (start 48 12.5) (end 41 19.5) (width 0.25) (layer F.Cu) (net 13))
 (via (at 39 32.5) (size 1.5) (drill 0.9) (layers F.Cu B.Cu) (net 32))
 (via (at 39 32.5) (size 1.5) (drill 0.9) (layers F.Cu B.Cu) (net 32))
 (segment (start 39 26.82) (end 39.25 26.57) (width 0.5) (layer F.Cu) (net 32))
 (segment (start 39 32.5) (end 39 26.82) (width 0.5) (layer F.Cu) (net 32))
 (segment (start 13.575001 35.924999) (end 35.575001 35.924999) (width 0.25) (layer B.Cu) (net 32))
 (segment (start 8.5 50.5) (end 8.5 41) (width 0.25) (layer B.Cu) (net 32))
 (segment (start 35.575001 35.924999) (end 39 32.5) (width 0.25) (layer B.Cu) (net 32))
 (segment (start 10.5 52.5) (end 8.5 50.5) (width 0.25) (layer B.Cu) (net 32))
 (segment (start 8.5 41) (end 13.575001 35.924999) (width 0.25) (layer B.Cu) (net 32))
 (segment (start 37.5 61.5) (end 37.5 54.5) (width 0.25) (layer F.Cu) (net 32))
 (via (at 37.5 54.5) (size 0.8) (drill 0.4) (layers F.Cu B.Cu) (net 32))
 (segment (start 37.5 54.5) (end 16 54.5) (width 0.25) (layer B.Cu) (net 32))
 (segment (start 16 54.5) (end 14 52.5) (width 0.25) (layer B.Cu) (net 32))
 (segment (start 14 52.5) (end 10.5 52.5) (width 0.25) (layer B.Cu) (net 32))
 (segment (start 6.5 61.5) (end 6.5 55) (width 0.25) (layer F.Cu) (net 15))
 (segment (start 6.5 48) (end 6.5 61.5) (width 0.25) (layer F.Cu) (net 15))
 (segment (start 14.5 40) (end 6.5 48) (width 0.25) (layer F.Cu) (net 15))
 (segment (start 44.5 40) (end 14.5 40) (width 0.25) (layer F.Cu) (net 15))
 (segment (start 49.41 44.91) (end 44.5 40) (width 0.25) (layer F.Cu) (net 15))
 (segment (start 49.41 46.89) (end 49.41 44.91) (width 0.25) (layer F.Cu) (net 15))
 (segment (start 46.87 44.87) (end 46.87 46.89) (width 0.25) (layer F.Cu) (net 16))
 (segment (start 43 41) (end 46.87 44.87) (width 0.25) (layer F.Cu) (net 16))
 (segment (start 14.5 41) (end 43 41) (width 0.25) (layer F.Cu) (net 16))
 (segment (start 8.5 47) (end 14.5 41) (width 0.25) (layer F.Cu) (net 16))
 (segment (start 8.5 61.5) (end 8.5 47) (width 0.25) (layer F.Cu) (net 16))
 (segment (start 44.33 46.89) (end 44.33 53.67) (width 0.5) (layer F.Cu) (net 17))
 (segment (start 43.5 54.5) (end 43.5 61.5) (width 0.5) (layer F.Cu) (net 17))
 (segment (start 44.33 53.67) (end 43.5 54.5) (width 0.5) (layer F.Cu) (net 17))
 (segment (start 41.79 46.89) (end 41.79 53.21) (width 0.5) (layer F.Cu) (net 18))
 (segment (start 41.5 53.5) (end 41.5 61.5) (width 0.5) (layer F.Cu) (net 18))
 (segment (start 41.79 53.21) (end 41.5 53.5) (width 0.5) (layer F.Cu) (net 18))
 (segment (start 39.25 46.89) (end 39.25 53.25) (width 0.5) (layer F.Cu) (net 19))
 (segment (start 39.5 53.5) (end 39.5 61.5) (width 0.5) (layer F.Cu) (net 19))
 (segment (start 39.25 53.25) (end 39.5 53.5) (width 0.5) (layer F.Cu) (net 19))
 (segment (start 10.5 61.5) (end 10.5 58.75) (width 0.5) (layer F.Cu) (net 21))
 (segment (start 34.17 44.67) (end 34.17 46.89) (width 0.25) (layer F.Cu) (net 21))
 (segment (start 32 42.5) (end 34.17 44.67) (width 0.25) (layer F.Cu) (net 21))
 (segment (start 10.5 46.5) (end 14.5 42.5) (width 0.25) (layer F.Cu) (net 21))
 (segment (start 10.5 54.5) (end 10.5 46.5) (width 0.25) (layer F.Cu) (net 21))
 (segment (start 14.5 42.5) (end 32 42.5) (width 0.25) (layer F.Cu) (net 21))
 (segment (start 10.5 61.5) (end 10.5 54.5) (width 0.25) (layer F.Cu) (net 21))
 (segment (start 10.5 54.5) (end 10.5 54) (width 0.25) (layer F.Cu) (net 21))
 (segment (start 26 61.5) (end 26 55) (width 0.5) (layer F.Cu) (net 23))
 (segment (start 29.09 51.91) (end 29.09 46.89) (width 0.5) (layer F.Cu) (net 23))
 (segment (start 26 55) (end 29.09 51.91) (width 0.5) (layer F.Cu) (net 23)))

